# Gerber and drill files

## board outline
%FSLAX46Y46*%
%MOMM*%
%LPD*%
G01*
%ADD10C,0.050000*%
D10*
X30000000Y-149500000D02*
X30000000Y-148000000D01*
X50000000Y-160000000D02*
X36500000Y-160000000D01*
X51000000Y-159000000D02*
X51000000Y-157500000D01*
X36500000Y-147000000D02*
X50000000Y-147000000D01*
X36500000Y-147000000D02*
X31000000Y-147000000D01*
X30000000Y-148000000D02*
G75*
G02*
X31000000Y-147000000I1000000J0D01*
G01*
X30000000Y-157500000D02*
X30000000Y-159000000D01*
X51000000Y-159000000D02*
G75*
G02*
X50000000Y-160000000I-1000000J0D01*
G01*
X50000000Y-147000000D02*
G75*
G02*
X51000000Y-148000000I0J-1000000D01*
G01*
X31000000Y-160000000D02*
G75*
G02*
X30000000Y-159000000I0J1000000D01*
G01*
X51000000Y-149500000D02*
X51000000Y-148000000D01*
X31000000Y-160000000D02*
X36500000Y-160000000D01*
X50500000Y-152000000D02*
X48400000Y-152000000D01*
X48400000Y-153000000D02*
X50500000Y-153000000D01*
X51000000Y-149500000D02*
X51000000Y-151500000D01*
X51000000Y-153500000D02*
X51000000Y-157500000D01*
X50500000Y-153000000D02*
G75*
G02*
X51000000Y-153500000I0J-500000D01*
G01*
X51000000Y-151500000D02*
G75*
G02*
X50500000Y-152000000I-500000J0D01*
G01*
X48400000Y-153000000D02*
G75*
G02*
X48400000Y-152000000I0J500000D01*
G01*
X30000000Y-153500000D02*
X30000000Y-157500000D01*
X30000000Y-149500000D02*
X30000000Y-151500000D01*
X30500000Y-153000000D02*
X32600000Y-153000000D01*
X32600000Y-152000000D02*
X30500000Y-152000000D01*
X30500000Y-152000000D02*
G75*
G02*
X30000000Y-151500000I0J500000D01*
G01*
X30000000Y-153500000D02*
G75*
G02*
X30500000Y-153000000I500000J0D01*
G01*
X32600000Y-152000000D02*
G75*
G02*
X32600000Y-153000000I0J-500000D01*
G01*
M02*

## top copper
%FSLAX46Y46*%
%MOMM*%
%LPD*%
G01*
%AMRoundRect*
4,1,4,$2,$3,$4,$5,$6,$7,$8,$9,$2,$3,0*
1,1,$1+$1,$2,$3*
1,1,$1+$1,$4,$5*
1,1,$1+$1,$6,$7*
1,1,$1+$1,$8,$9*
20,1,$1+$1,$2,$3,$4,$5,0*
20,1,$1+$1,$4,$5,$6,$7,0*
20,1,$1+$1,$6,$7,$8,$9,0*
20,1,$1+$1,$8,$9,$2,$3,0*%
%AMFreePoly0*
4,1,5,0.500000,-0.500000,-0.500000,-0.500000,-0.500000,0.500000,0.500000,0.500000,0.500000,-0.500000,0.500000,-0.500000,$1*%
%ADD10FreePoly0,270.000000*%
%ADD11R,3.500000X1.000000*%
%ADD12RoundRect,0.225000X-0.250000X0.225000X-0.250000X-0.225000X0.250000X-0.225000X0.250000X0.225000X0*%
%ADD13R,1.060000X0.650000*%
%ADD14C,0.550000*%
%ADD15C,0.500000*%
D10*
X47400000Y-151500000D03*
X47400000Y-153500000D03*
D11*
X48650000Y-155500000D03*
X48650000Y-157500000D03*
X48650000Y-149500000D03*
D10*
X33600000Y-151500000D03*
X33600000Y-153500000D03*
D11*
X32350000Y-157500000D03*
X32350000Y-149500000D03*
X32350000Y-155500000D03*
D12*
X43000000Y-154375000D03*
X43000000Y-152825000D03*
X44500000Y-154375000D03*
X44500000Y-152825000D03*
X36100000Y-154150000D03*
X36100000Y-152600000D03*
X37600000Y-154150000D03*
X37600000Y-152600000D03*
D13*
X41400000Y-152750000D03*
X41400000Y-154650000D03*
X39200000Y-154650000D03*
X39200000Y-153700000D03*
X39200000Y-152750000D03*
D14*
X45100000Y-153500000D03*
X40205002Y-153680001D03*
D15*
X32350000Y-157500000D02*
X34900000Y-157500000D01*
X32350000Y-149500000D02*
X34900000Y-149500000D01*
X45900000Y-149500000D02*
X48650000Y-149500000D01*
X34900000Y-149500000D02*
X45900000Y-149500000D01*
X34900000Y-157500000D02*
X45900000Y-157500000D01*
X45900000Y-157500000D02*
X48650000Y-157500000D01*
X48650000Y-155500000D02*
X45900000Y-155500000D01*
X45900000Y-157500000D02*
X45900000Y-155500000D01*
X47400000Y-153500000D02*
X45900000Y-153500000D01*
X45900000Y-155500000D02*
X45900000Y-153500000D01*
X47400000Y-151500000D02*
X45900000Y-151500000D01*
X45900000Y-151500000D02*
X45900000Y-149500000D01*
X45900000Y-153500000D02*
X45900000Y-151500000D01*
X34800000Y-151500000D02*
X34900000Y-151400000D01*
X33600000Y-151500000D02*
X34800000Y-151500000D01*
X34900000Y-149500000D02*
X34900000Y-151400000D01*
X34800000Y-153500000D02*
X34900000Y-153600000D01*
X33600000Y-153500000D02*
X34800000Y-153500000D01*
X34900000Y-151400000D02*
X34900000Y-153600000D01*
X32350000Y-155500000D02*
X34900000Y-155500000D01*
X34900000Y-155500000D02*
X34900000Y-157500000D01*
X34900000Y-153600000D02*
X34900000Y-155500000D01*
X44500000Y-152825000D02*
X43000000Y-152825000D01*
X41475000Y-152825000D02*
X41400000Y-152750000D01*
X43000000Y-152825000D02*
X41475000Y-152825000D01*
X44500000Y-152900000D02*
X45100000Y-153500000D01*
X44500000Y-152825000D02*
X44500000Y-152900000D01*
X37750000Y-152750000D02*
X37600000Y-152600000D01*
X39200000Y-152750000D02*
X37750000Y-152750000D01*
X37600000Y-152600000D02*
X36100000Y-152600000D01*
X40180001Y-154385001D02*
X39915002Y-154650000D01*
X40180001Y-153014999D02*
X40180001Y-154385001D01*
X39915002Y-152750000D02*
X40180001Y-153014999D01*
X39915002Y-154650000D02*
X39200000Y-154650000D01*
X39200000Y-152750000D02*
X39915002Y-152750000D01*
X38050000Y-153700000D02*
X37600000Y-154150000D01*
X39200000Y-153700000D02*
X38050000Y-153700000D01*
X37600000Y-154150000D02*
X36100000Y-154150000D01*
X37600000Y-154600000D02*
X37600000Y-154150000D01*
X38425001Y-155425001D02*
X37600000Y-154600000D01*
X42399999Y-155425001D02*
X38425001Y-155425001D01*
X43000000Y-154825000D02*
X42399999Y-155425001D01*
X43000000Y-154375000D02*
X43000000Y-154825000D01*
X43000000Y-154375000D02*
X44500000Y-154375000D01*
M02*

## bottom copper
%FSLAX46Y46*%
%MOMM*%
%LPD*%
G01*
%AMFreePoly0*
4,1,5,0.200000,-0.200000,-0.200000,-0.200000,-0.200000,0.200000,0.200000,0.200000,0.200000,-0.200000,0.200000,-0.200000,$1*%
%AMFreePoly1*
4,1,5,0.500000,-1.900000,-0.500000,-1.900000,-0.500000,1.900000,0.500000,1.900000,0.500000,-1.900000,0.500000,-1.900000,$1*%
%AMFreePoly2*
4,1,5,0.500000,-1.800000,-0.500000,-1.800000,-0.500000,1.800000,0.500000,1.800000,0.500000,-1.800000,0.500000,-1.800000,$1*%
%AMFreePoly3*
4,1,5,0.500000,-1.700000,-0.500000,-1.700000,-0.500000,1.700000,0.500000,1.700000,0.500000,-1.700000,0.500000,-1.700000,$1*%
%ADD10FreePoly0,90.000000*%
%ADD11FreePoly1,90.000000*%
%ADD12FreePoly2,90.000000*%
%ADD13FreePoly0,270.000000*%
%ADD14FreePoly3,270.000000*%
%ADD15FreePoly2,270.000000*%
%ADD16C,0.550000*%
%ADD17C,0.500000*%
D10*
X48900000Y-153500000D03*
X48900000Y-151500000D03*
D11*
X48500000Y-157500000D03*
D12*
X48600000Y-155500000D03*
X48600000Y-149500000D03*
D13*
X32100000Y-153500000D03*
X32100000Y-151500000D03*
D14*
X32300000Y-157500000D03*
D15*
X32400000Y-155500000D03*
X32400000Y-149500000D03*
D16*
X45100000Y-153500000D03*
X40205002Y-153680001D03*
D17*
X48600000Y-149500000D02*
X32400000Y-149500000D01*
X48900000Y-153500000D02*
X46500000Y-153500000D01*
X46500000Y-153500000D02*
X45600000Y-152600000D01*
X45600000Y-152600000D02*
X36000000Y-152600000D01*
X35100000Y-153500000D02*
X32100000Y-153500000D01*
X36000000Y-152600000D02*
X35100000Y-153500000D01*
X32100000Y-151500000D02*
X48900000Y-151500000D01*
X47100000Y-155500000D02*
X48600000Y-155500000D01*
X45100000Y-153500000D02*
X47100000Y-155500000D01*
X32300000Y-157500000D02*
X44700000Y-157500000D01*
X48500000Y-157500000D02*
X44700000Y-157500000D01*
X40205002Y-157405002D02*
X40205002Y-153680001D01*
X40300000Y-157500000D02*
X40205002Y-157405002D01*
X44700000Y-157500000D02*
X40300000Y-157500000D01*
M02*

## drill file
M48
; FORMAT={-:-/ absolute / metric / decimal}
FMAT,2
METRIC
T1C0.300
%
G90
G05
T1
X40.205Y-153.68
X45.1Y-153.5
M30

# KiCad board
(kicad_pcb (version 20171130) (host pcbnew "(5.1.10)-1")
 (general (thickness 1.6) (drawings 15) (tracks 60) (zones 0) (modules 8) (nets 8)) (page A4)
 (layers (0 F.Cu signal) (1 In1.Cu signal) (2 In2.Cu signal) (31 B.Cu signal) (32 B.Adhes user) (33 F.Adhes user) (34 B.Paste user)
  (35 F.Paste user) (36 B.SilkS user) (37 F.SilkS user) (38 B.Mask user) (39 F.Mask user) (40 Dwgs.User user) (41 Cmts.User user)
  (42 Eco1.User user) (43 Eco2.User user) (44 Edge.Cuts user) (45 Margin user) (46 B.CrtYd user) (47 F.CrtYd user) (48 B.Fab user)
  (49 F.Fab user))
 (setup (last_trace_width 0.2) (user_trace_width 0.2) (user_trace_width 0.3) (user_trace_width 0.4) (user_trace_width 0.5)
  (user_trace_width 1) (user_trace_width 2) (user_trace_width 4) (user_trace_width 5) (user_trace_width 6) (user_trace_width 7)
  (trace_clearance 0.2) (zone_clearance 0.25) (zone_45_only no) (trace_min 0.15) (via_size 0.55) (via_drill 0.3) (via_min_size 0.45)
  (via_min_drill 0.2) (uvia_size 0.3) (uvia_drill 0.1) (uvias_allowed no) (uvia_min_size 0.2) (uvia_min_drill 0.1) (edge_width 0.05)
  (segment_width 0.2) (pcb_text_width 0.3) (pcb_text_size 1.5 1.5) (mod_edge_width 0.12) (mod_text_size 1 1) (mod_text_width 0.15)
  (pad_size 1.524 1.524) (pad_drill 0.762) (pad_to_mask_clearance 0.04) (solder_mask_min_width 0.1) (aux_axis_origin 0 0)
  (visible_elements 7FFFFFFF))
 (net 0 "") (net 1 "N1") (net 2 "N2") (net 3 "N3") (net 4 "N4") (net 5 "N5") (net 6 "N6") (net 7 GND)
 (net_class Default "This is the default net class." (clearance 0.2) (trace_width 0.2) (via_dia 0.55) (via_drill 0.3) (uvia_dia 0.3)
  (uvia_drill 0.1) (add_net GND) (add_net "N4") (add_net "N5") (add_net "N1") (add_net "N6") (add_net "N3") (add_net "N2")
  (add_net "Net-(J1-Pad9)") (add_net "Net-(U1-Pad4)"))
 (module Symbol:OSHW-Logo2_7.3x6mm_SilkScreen (layer B.Cu) (at 40.4 157.1 180)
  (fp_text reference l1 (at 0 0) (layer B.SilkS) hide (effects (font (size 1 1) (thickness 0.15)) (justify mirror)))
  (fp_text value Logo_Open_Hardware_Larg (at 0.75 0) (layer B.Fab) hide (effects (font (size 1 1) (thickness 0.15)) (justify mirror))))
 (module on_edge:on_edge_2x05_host (layer F.Cu) (at 51 153.5 270)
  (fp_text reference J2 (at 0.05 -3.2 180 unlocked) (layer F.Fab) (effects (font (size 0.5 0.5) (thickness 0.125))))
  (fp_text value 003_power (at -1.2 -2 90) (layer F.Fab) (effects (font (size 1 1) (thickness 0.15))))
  (fp_line (start -1.5 0.5) (end -1.5 2.6) (layer Edge.Cuts) (width 0.05))
  (fp_line (start -0.5 2.6) (end -0.5 0.5) (layer Edge.Cuts) (width 0.05))
  (fp_line (start -4 0) (end -2 0) (layer Edge.Cuts) (width 0.05))
  (fp_line (start 0 0) (end 4 0) (layer Edge.Cuts) (width 0.05))
  (fp_arc (start 0 0.5) (end 0 0) (angle -90) (layer Edge.Cuts) (width 0.05))
  (fp_arc (start -2 0.5) (end -1.5 0.5) (angle -90) (layer Edge.Cuts) (width 0.05))
  (fp_arc (start -1 2.6) (end -1.5 2.6) (angle -180) (layer Edge.Cuts) (width 0.05))
  (pad 2 smd custom (at -2 3.6 270) (size 1 1) (layers F.Cu F.Mask) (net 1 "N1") (zone_connect 0)
   (options (clearance outline) (anchor rect)) (primitives))
  (pad 3 smd custom (at 0 3.6 270) (size 1 1) (layers F.Cu F.Mask) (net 1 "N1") (zone_connect 0) (options (clearance outline) (anchor rect))
   (primitives))
  (pad 8 smd custom (at 0 2.1 90) (size 0.4 0.4) (layers B.Cu B.Mask) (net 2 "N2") (zone_connect 0)
   (options (clearance outline) (anchor rect)) (primitives))
  (pad 7 smd custom (at -2 2.1 90) (size 0.4 0.4) (layers B.Cu B.Mask) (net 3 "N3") (zone_connect 0)
   (options (clearance outline) (anchor rect)) (primitives))
  (pad 4 smd rect (at 2 2.35 270) (size 1 3.5) (layers F.Cu F.Mask) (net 1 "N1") (zone_connect 0))
  (pad 10 smd custom (at 4 2.5 90) (size 1 3.8) (layers B.Cu B.Mask) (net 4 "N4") (zone_connect 0)
   (options (clearance outline) (anchor rect)) (primitives))
  (pad 9 smd custom (at 2 2.4 90) (size 1 3.6) (layers B.Cu B.Mask) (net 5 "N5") (zone_connect 0)
   (options (clearance outline) (anchor rect)) (primitives))
  (pad 6 smd custom (at -4 2.4 90) (size 1 3.6) (layers B.Cu B.Mask) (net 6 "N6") (zone_connect 0)
   (options (clearance outline) (anchor rect)) (primitives))
  (pad 5 smd rect (at 4 2.35 270) (size 1 3.5) (layers F.Cu F.Mask) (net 1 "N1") (zone_connect 0))
  (pad 1 smd rect (at -4 2.35 270) (size 1 3.5) (layers F.Cu F.Mask) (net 1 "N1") (zone_connect 0)))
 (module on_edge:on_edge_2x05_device (layer F.Cu) (at 30 153.5 270)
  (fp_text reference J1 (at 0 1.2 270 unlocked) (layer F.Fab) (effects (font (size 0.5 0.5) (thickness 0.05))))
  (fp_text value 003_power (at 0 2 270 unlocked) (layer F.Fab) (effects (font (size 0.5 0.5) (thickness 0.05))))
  (fp_line (start 0 0) (end 4 0) (layer Edge.Cuts) (width 0.05))
  (fp_line (start -4 0) (end -2 0) (layer Edge.Cuts) (width 0.05))
  (fp_line (start -0.5 -0.5) (end -0.5 -2.6) (layer Edge.Cuts) (width 0.05))
  (fp_line (start -1.5 -2.6) (end -1.5 -0.5) (layer Edge.Cuts) (width 0.05))
  (fp_arc (start -2 -0.5) (end -2 0) (angle -90) (layer Edge.Cuts) (width 0.05))
  (fp_arc (start 0 -0.5) (end -0.5 -0.5) (angle -90) (layer Edge.Cuts) (width 0.05))
  (fp_arc (start -1 -2.6) (end -0.5 -2.6) (angle -180) (layer Edge.Cuts) (width 0.05))
  (pad 2 smd custom (at -2 -3.6 270) (size 1 1) (layers F.Cu F.Mask) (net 1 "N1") (zone_connect 0)
   (options (clearance outline) (anchor rect)) (primitives))
  (pad 3 smd custom (at 0 -3.6 270) (size 1 1) (layers F.Cu F.Mask) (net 1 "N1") (zone_connect 0)
   (options (clearance outline) (anchor rect)) (primitives))
  (pad 8 smd custom (at 0 -2.1 270) (size 0.4 0.4) (layers B.Cu B.Mask) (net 2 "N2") (zone_connect 0)
   (options (clearance outline) (anchor rect)) (primitives))
  (pad 7 smd custom (at -2 -2.1 270) (size 0.4 0.4) (layers B.Cu B.Mask) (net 3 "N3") (zone_connect 0)
   (options (clearance outline) (anchor rect)) (primitives))
  (pad 10 smd custom (at 4 -2.3 270) (size 1 3.4) (layers B.Cu B.Mask) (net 4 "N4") (zone_connect 0)
   (options (clearance outline) (anchor rect)) (primitives))
  (pad 9 smd custom (at 2 -2.4 270) (size 1 3.6) (layers B.Cu B.Mask) (zone_connect 0) (options (clearance outline) (anchor rect))
   (primitives))
  (pad 6 smd custom (at -4 -2.4 270) (size 1 3.6) (layers B.Cu B.Mask) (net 6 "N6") (zone_connect 0)
   (options (clearance outline) (anchor rect)) (primitives))
  (pad 5 smd rect (at 4 -2.35 90) (size 1 3.5) (layers F.Cu F.Mask) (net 1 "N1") (zone_connect 0))
  (pad 1 smd rect (at -4 -2.35 90) (size 1 3.5) (layers F.Cu F.Mask) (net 1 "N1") (zone_connect 0))
  (pad 4 smd rect (at 2 -2.35 90) (size 1 3.5) (layers F.Cu F.Mask) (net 1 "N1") (zone_connect 0)))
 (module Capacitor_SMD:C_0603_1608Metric (layer F.Cu) (at 43 153.6 270)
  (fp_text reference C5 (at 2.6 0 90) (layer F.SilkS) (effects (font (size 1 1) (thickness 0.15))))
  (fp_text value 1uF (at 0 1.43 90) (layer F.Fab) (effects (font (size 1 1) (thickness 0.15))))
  (pad 2 smd roundrect (at 0.775 0 270) (size 0.9 0.95) (layers F.Cu F.Paste F.Mask) (roundrect_rratio 0.25) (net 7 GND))
  (pad 1 smd roundrect (at -0.775 0 270) (size 0.9 0.95) (layers F.Cu F.Paste F.Mask) (roundrect_rratio 0.25) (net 5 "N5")))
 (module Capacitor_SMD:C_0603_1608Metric (layer F.Cu) (at 44.5 153.6 270)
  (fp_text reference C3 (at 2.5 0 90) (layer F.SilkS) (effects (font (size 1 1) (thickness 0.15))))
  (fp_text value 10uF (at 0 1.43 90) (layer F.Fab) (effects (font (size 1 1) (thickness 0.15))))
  (pad 2 smd roundrect (at 0.775 0 270) (size 0.9 0.95) (layers F.Cu F.Paste F.Mask) (roundrect_rratio 0.25) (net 7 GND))
  (pad 1 smd roundrect (at -0.775 0 270) (size 0.9 0.95) (layers F.Cu F.Paste F.Mask) (roundrect_rratio 0.25) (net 5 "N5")))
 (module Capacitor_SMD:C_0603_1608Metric (layer F.Cu) (at 36.1 153.375 270)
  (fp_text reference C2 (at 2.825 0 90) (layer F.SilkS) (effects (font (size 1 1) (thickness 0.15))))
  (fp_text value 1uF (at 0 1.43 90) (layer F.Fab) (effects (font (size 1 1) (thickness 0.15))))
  (pad 2 smd roundrect (at 0.775 0 270) (size 0.9 0.95) (layers F.Cu F.Paste F.Mask) (roundrect_rratio 0.25) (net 7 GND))
  (pad 1 smd roundrect (at -0.775 0 270) (size 0.9 0.95) (layers F.Cu F.Paste F.Mask) (roundrect_rratio 0.25) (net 4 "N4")))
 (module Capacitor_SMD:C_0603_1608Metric (layer F.Cu) (at 37.6 153.375 270)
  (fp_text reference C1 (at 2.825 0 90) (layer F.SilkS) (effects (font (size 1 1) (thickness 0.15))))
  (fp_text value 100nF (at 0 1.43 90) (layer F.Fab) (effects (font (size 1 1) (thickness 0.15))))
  (pad 2 smd roundrect (at 0.775 0 270) (size 0.9 0.95) (layers F.Cu F.Paste F.Mask) (roundrect_rratio 0.25) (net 7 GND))
  (pad 1 smd roundrect (at -0.775 0 270) (size 0.9 0.95) (layers F.Cu F.Paste F.Mask) (roundrect_rratio 0.25) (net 4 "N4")))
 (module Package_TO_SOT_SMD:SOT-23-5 (layer F.Cu) (at 40.3 153.7)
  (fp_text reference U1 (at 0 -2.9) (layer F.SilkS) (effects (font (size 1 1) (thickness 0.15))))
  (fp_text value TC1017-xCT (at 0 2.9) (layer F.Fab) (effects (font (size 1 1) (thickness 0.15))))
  (pad 5 smd rect (at 1.1 -0.95) (size 1.06 0.65) (layers F.Cu F.Paste F.Mask) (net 5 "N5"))
  (pad 4 smd rect (at 1.1 0.95) (size 1.06 0.65) (layers F.Cu F.Paste F.Mask))
  (pad 3 smd rect (at -1.1 0.95) (size 1.06 0.65) (layers F.Cu F.Paste F.Mask) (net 4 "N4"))
  (pad 2 smd rect (at -1.1 0) (size 1.06 0.65) (layers F.Cu F.Paste F.Mask) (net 7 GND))
  (pad 1 smd rect (at -1.1 -0.95) (size 1.06 0.65) (layers F.Cu F.Paste F.Mask) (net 4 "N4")))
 (gr_line (start 30 149.5) (end 30 148) (layer Edge.Cuts) (width 0.05))
 (gr_line (start 50 160) (end 36.5 160) (layer Edge.Cuts) (width 0.05))
 (gr_line (start 51 159) (end 51 157.5) (layer Edge.Cuts) (width 0.05))
 (gr_line (start 36.5 147) (end 50 147) (layer Edge.Cuts) (width 0.05))
 (gr_line (start 36.5 147) (end 31 147) (layer Edge.Cuts) (width 0.05))
 (gr_arc (start 31 148) (end 31 147) (angle -90) (layer Edge.Cuts) (width 0.05))
 (gr_line (start 30 157.5) (end 30 159) (layer Edge.Cuts) (width 0.05))
 (gr_arc (start 50 159) (end 50 160) (angle -90) (layer Edge.Cuts) (width 0.05))
 (gr_arc (start 50 148) (end 51 148) (angle -90) (layer Edge.Cuts) (width 0.05))
 (gr_arc (start 31 159) (end 30 159) (angle -90) (layer Edge.Cuts) (width 0.05))
 (gr_line (start 51 149.5) (end 51 148) (layer Edge.Cuts) (width 0.05))
 (gr_line (start 31 160) (end 36.5 160) (layer Edge.Cuts) (width 0.05))
 (segment (start 32.35 157.5) (end 34.9 157.5) (width 0.5) (layer F.Cu) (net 1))
 (segment (start 32.35 149.5) (end 34.9 149.5) (width 0.5) (layer F.Cu) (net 1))
 (segment (start 45.9 149.5) (end 48.65 149.5) (width 0.5) (layer F.Cu) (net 1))
 (segment (start 34.9 149.5) (end 45.9 149.5) (width 0.5) (layer F.Cu) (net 1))
 (segment (start 34.9 157.5) (end 45.9 157.5) (width 0.5) (layer F.Cu) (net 1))
 (segment (start 45.9 157.5) (end 48.65 157.5) (width 0.5) (layer F.Cu) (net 1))
 (segment (start 48.65 155.5) (end 45.9 155.5) (width 0.5) (layer F.Cu) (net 1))
 (segment (start 45.9 157.5) (end 45.9 155.5) (width 0.5) (layer F.Cu) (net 1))
 (segment (start 47.4 153.5) (end 45.9 153.5) (width 0.5) (layer F.Cu) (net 1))
 (segment (start 45.9 155.5) (end 45.9 153.5) (width 0.5) (layer F.Cu) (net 1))
 (segment (start 47.4 151.5) (end 45.9 151.5) (width 0.5) (layer F.Cu) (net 1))
 (segment (start 45.9 151.5) (end 45.9 149.5) (width 0.5) (layer F.Cu) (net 1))
 (segment (start 45.9 153.5) (end 45.9 151.5) (width 0.5) (layer F.Cu) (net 1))
 (segment (start 34.8 151.5) (end 34.9 151.4) (width 0.5) (layer F.Cu) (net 1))
 (segment (start 33.6 151.5) (end 34.8 151.5) (width 0.5) (layer F.Cu) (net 1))
 (segment (start 34.9 149.5) (end 34.9 151.4) (width 0.5) (layer F.Cu) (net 1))
 (segment (start 34.8 153.5) (end 34.9 153.6) (width 0.5) (layer F.Cu) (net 1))
 (segment (start 33.6 153.5) (end 34.8 153.5) (width 0.5) (layer F.Cu) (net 1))
 (segment (start 34.9 151.4) (end 34.9 153.6) (width 0.5) (layer F.Cu) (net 1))
 (segment (start 32.35 155.5) (end 34.9 155.5) (width 0.5) (layer F.Cu) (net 1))
 (segment (start 34.9 155.5) (end 34.9 157.5) (width 0.5) (layer F.Cu) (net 1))
 (segment (start 34.9 153.6) (end 34.9 155.5) (width 0.5) (layer F.Cu) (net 1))
 (segment (start 48.6 149.5) (end 32.4 149.5) (width 0.5) (layer B.Cu) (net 6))
 (segment (start 48.9 153.5) (end 46.5 153.5) (width 0.5) (layer B.Cu) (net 2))
 (segment (start 46.5 153.5) (end 45.6 152.6) (width 0.5) (layer B.Cu) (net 2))
 (segment (start 45.6 152.6) (end 36 152.6) (width 0.5) (layer B.Cu) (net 2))
 (segment (start 35.1 153.5) (end 32.1 153.5) (width 0.5) (layer B.Cu) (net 2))
 (segment (start 36 152.6) (end 35.1 153.5) (width 0.5) (layer B.Cu) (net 2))
 (segment (start 32.1 151.5) (end 48.9 151.5) (width 0.5) (layer B.Cu) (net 3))
 (segment (start 44.5 152.825) (end 43 152.825) (width 0.5) (layer F.Cu) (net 5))
 (segment (start 41.475 152.825) (end 41.4 152.75) (width 0.5) (layer F.Cu) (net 5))
 (segment (start 43 152.825) (end 41.475 152.825) (width 0.5) (layer F.Cu) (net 5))
 (via (at 45.1 153.5) (size 0.55) (drill 0.3) (layers F.Cu B.Cu) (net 5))
 (segment (start 44.5 152.9) (end 45.1 153.5) (width 0.5) (layer F.Cu) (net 5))
 (segment (start 44.5 152.825) (end 44.5 152.9) (width 0.5) (layer F.Cu) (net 5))
 (segment (start 47.1 155.5) (end 48.6 155.5) (width 0.5) (layer B.Cu) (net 5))
 (segment (start 45.1 153.5) (end 47.1 155.5) (width 0.5) (layer B.Cu) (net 5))
 (segment (start 37.75 152.75) (end 37.6 152.6) (width 0.5) (layer F.Cu) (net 4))
 (segment (start 39.2 152.75) (end 37.75 152.75) (width 0.5) (layer F.Cu) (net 4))
 (segment (start 37.6 152.6) (end 36.1 152.6) (width 0.5) (layer F.Cu) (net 4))
 (segment (start 40.180001 154.385001) (end 39.915002 154.65) (width 0.5) (layer F.Cu) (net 4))
 (segment (start 40.180001 153.014999) (end 40.180001 154.385001) (width 0.5) (layer F.Cu) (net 4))
 (segment (start 39.915002 152.75) (end 40.180001 153.014999) (width 0.5) (layer F.Cu) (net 4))
 (segment (start 39.915002 154.65) (end 39.2 154.65) (width 0.5) (layer F.Cu) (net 4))
 (segment (start 39.2 152.75) (end 39.915002 152.75) (width 0.5) (layer F.Cu) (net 4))
 (via (at 40.205002 153.680001) (size 0.55) (drill 0.3) (layers F.Cu B.Cu) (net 4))
 (segment (start 32.3 157.5) (end 44.7 157.5) (width 0.5) (layer B.Cu) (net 4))
 (segment (start 48.5 157.5) (end 44.7 157.5) (width 0.5) (layer B.Cu) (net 4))
 (segment (start 40.205002 157.405002) (end 40.205002 153.680001) (width 0.5) (layer B.Cu) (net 4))
 (segment (start 40.3 157.5) (end 40.205002 157.405002) (width 0.5) (layer B.Cu) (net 4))
 (segment (start 44.7 157.5) (end 40.3 157.5) (width 0.5) (layer B.Cu) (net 4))
 (segment (start 38.05 153.7) (end 37.6 154.15) (width 0.5) (layer F.Cu) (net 7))
 (segment (start 39.2 153.7) (end 38.05 153.7) (width 0.5) (layer F.Cu) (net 7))
 (segment (start 37.6 154.15) (end 36.1 154.15) (width 0.5) (layer F.Cu) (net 7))
 (segment (start 37.6 154.6) (end 37.6 154.15) (width 0.5) (layer F.Cu) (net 7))
 (segment (start 38.425001 155.425001) (end 37.6 154.6) (width 0.5) (layer F.Cu) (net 7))
 (segment (start 42.399999 155.425001) (end 38.425001 155.425001) (width 0.5) (layer F.Cu) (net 7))
 (segment (start 43 154.825) (end 42.399999 155.425001) (width 0.5) (layer F.Cu) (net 7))
 (segment (start 43 154.375) (end 43 154.825) (width 0.5) (layer F.Cu) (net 7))
 (segment (start 43 154.375) (end 44.5 154.375) (width 0.5) (layer F.Cu) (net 7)))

